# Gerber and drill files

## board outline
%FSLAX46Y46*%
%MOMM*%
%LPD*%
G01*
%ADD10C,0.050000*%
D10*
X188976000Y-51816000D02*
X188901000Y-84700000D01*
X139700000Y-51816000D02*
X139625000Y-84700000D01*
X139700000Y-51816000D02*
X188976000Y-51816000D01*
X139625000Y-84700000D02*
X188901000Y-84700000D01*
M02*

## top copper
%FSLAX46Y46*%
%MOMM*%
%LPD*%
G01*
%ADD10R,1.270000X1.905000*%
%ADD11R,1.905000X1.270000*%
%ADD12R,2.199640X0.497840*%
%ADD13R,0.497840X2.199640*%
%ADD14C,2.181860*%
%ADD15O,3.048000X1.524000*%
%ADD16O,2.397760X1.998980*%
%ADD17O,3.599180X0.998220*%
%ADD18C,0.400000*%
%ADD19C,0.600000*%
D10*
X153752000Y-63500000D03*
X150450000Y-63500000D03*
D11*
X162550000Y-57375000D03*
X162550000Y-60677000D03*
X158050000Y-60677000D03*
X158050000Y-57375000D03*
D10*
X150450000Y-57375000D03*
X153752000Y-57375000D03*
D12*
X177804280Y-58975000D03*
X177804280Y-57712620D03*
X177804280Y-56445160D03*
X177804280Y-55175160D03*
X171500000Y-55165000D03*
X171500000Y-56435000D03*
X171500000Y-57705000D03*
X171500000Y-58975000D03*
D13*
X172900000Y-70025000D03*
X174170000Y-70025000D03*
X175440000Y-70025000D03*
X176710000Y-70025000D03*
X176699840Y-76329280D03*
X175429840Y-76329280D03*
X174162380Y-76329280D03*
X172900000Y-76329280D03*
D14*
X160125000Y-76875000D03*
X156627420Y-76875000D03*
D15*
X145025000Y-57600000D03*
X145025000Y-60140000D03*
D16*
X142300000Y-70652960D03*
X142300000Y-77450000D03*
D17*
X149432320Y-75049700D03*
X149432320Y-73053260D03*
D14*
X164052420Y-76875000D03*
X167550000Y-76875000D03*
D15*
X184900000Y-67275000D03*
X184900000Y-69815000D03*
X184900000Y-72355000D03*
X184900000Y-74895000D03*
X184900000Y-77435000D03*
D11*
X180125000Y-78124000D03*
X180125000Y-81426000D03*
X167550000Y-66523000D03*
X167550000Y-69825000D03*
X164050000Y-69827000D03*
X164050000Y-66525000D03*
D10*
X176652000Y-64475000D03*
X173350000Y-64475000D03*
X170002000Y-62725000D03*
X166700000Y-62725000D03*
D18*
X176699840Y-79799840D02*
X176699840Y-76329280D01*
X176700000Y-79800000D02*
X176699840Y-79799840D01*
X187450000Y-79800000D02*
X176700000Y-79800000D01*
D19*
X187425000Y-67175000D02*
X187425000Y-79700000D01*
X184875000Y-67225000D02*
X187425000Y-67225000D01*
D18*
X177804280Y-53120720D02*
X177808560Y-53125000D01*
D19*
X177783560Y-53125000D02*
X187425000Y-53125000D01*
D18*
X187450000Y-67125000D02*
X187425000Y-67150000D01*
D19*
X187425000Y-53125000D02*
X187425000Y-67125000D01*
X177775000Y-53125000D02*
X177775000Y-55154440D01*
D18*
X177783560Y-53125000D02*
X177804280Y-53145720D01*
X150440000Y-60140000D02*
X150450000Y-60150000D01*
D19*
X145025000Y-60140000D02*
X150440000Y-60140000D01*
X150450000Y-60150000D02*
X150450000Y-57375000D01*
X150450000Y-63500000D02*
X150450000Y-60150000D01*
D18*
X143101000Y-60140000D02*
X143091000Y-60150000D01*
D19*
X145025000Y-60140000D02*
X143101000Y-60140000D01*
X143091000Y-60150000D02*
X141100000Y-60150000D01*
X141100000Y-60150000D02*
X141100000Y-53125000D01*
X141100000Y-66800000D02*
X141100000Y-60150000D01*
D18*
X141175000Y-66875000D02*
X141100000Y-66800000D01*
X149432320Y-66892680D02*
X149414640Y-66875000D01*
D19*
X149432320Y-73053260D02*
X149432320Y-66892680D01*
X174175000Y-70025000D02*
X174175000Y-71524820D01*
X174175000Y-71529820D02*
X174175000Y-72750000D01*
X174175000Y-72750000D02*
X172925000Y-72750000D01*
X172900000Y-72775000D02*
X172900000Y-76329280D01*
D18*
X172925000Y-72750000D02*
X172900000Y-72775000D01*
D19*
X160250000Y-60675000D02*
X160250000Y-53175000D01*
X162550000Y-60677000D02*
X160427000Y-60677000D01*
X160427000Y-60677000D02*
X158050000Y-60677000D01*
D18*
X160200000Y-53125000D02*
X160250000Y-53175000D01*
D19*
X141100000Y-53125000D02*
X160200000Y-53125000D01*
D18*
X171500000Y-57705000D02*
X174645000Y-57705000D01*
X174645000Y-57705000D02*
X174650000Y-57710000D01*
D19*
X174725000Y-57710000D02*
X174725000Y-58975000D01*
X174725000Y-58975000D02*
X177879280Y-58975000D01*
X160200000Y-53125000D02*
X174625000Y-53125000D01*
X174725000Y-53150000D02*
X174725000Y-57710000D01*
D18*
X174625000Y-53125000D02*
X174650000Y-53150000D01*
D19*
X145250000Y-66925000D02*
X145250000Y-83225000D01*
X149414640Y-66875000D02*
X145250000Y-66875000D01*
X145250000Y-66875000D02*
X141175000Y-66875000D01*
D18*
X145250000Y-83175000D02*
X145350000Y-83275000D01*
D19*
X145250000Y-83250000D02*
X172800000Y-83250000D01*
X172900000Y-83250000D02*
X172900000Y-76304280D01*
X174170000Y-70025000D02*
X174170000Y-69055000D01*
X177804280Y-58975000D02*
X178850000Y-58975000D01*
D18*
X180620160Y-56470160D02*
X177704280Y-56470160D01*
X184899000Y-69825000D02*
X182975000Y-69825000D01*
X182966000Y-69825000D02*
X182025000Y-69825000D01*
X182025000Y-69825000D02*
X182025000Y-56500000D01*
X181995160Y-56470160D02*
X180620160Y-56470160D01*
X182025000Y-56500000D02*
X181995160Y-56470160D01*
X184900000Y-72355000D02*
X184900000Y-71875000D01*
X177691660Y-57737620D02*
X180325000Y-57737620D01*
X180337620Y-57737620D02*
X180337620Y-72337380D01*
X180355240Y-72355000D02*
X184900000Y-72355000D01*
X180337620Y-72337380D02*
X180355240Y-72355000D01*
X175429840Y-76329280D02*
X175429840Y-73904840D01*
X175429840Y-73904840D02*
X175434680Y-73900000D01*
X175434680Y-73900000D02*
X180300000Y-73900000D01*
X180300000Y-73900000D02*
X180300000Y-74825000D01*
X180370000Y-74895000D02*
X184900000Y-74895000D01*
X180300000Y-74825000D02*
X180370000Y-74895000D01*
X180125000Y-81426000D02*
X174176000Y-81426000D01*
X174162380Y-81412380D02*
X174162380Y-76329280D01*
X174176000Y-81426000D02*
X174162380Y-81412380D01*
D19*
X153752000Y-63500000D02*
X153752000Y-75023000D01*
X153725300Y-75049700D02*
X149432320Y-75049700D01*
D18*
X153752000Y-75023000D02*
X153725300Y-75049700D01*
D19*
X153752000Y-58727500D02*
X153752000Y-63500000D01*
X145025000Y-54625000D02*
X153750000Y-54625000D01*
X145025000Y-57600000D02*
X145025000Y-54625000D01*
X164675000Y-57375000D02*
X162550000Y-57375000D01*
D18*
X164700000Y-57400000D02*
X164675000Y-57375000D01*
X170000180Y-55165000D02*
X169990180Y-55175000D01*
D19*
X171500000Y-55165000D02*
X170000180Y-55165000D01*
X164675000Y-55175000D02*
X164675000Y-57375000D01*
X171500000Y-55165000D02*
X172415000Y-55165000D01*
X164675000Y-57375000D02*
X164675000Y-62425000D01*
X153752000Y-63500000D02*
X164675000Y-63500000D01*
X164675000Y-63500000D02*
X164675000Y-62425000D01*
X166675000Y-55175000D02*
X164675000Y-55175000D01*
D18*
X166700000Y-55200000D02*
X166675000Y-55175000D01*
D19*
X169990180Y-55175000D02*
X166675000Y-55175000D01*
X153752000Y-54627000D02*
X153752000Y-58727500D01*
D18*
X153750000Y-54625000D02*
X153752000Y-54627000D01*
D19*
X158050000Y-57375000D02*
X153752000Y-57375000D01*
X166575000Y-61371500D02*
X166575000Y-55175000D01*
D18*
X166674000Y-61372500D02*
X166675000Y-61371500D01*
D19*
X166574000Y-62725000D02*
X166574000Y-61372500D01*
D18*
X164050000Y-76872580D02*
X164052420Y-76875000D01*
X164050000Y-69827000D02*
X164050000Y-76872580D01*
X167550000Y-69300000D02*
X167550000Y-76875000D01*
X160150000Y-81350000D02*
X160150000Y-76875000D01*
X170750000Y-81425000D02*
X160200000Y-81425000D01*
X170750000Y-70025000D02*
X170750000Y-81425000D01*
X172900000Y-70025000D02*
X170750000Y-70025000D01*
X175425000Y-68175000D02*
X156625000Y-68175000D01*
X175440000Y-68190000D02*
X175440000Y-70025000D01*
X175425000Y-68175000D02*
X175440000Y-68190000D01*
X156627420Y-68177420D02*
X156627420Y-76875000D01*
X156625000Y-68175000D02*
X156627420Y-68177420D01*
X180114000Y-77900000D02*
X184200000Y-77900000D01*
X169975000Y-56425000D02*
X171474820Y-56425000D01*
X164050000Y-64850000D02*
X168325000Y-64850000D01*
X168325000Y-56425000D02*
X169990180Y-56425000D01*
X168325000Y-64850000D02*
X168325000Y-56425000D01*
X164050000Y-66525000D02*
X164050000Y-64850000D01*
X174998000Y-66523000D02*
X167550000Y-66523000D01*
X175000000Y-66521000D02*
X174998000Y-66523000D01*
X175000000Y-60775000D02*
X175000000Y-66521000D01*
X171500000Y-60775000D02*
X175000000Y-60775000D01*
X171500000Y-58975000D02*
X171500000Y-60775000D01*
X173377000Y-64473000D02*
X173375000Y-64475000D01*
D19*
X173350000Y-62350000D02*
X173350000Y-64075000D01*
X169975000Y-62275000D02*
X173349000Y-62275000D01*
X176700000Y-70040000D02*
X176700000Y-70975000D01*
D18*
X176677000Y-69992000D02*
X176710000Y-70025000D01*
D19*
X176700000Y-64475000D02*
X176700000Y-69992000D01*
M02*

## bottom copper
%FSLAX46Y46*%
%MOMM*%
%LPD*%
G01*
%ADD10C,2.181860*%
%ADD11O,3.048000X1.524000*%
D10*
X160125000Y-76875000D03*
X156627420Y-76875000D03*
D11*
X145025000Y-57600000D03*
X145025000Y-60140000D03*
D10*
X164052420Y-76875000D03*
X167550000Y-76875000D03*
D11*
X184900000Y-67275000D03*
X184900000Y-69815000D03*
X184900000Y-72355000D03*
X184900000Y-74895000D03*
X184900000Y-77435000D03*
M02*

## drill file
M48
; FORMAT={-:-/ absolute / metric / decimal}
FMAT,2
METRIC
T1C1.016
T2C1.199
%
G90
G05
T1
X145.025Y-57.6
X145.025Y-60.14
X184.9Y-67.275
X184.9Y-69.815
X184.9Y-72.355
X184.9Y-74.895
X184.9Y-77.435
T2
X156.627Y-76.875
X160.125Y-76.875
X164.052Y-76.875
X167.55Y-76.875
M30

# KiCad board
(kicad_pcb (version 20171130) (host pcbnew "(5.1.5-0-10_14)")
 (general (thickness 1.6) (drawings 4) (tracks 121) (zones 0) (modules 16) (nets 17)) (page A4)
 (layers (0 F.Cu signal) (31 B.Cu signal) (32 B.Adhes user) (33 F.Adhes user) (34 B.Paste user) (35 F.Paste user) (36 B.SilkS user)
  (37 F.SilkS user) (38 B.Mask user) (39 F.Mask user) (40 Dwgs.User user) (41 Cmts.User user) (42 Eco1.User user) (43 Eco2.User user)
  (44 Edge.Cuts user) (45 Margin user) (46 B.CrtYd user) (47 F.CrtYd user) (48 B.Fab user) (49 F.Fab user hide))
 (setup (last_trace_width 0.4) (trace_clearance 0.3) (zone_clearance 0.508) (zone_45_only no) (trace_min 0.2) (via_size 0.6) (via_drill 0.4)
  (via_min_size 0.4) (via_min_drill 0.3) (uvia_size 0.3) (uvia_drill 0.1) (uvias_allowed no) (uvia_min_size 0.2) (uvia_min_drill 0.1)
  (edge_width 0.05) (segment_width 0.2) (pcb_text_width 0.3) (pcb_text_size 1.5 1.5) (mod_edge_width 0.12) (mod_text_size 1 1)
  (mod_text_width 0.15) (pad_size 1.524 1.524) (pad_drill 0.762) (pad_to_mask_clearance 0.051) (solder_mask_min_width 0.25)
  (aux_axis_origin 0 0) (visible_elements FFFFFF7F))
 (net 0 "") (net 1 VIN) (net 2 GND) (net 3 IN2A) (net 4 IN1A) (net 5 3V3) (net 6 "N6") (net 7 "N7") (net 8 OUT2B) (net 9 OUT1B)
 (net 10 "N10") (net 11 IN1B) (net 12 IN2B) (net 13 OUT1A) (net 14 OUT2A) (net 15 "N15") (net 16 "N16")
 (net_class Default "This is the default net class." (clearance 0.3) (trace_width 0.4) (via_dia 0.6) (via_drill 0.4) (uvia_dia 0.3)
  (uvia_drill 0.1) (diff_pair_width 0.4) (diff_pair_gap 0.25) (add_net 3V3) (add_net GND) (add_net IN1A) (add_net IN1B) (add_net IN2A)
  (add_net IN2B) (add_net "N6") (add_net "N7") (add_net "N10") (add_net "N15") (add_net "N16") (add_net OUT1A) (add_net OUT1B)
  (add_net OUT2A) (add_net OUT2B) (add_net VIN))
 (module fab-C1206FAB (layer F.Cu) (at 152.101 63.5 180)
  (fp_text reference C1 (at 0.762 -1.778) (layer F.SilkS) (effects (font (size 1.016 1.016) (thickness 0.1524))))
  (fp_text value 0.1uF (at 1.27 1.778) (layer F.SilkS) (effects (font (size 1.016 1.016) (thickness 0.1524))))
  (pad 1 smd rect (at -1.651 0 180) (size 1.27 1.905) (layers F.Cu F.Paste F.Mask) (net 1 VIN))
  (pad 2 smd rect (at 1.651 0 180) (size 1.27 1.905) (layers F.Cu F.Paste F.Mask) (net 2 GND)))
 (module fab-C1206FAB (layer F.Cu) (at 162.55 59.026 270)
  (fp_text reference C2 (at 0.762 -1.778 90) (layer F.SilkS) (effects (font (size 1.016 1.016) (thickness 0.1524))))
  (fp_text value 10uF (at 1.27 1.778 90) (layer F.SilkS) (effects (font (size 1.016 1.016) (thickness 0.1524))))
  (pad 1 smd rect (at -1.651 0 270) (size 1.27 1.905) (layers F.Cu F.Paste F.Mask) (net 1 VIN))
  (pad 2 smd rect (at 1.651 0 270) (size 1.27 1.905) (layers F.Cu F.Paste F.Mask) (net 2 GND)))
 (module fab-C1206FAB (layer F.Cu) (at 158.05 59.026 270)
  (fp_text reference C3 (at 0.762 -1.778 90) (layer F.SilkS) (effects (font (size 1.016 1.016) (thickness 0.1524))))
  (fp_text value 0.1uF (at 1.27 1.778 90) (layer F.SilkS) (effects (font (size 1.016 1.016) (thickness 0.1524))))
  (pad 2 smd rect (at 1.651 0 270) (size 1.27 1.905) (layers F.Cu F.Paste F.Mask) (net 2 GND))
  (pad 1 smd rect (at -1.651 0 270) (size 1.27 1.905) (layers F.Cu F.Paste F.Mask) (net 1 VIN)))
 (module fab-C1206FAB (layer F.Cu) (at 152.101 57.375 180)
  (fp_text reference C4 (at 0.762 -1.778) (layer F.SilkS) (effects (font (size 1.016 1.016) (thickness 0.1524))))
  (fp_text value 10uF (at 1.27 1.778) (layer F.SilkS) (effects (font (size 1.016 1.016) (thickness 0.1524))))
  (pad 2 smd rect (at 1.651 0 180) (size 1.27 1.905) (layers F.Cu F.Paste F.Mask) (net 2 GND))
  (pad 1 smd rect (at -1.651 0 180) (size 1.27 1.905) (layers F.Cu F.Paste F.Mask) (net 1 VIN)))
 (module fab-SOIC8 (layer F.Cu) (at 174.65214 57.07 90)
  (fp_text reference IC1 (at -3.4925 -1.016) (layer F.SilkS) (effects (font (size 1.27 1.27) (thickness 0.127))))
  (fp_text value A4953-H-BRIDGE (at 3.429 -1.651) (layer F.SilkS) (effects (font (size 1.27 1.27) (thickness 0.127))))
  (pad 1 smd rect (at -1.905 3.15214 90) (size 0.49784 2.19964) (layers F.Cu F.Paste F.Mask) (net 2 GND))
  (pad 2 smd rect (at -0.64262 3.15214 90) (size 0.49784 2.19964) (layers F.Cu F.Paste F.Mask) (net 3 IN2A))
  (pad 3 smd rect (at 0.62484 3.15214 90) (size 0.49784 2.19964) (layers F.Cu F.Paste F.Mask) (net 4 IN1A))
  (pad 4 smd rect (at 1.89484 3.15214 90) (size 0.49784 2.19964) (layers F.Cu F.Paste F.Mask) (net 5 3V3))
  (pad 5 smd rect (at 1.905 -3.15214 90) (size 0.49784 2.19964) (layers F.Cu F.Paste F.Mask) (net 1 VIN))
  (pad 6 smd rect (at 0.635 -3.15214 90) (size 0.49784 2.19964) (layers F.Cu F.Paste F.Mask) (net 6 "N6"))
  (pad 7 smd rect (at -0.635 -3.15214 90) (size 0.49784 2.19964) (layers F.Cu F.Paste F.Mask) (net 2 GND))
  (pad 8 smd rect (at -1.905 -3.15214 90) (size 0.49784 2.19964) (layers F.Cu F.Paste F.Mask) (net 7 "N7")))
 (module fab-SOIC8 (layer F.Cu) (at 174.805 73.17714)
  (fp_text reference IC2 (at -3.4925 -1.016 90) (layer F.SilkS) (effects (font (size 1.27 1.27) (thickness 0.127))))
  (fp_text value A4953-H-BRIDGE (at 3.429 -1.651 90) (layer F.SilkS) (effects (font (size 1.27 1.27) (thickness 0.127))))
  (pad 8 smd rect (at -1.905 -3.15214) (size 0.49784 2.19964) (layers F.Cu F.Paste F.Mask) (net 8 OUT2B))
  (pad 7 smd rect (at -0.635 -3.15214) (size 0.49784 2.19964) (layers F.Cu F.Paste F.Mask) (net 2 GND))
  (pad 6 smd rect (at 0.635 -3.15214) (size 0.49784 2.19964) (layers F.Cu F.Paste F.Mask) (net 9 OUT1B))
  (pad 5 smd rect (at 1.905 -3.15214) (size 0.49784 2.19964) (layers F.Cu F.Paste F.Mask) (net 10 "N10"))
  (pad 4 smd rect (at 1.89484 3.15214) (size 0.49784 2.19964) (layers F.Cu F.Paste F.Mask) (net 5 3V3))
  (pad 3 smd rect (at 0.62484 3.15214) (size 0.49784 2.19964) (layers F.Cu F.Paste F.Mask) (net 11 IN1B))
  (pad 2 smd rect (at -0.64262 3.15214) (size 0.49784 2.19964) (layers F.Cu F.Paste F.Mask) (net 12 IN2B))
  (pad 1 smd rect (at -1.905 3.15214) (size 0.49784 2.19964) (layers F.Cu F.Paste F.Mask) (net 2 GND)))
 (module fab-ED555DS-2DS (layer F.Cu) (at 158.32668 76.875)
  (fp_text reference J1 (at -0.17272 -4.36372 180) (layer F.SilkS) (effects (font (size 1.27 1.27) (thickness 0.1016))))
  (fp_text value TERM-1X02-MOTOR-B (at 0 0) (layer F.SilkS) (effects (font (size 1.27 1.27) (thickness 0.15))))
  (pad 1 thru_hole circle (at 1.79832 0) (size 2.18186 2.18186) (drill 1.19888) (layers F&B.Cu F.Paste F.SilkS F.Mask) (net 8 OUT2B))
  (pad 2 thru_hole circle (at -1.69926 0) (size 2.18186 2.18186) (drill 1.19888) (layers F&B.Cu F.Paste F.SilkS F.Mask) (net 9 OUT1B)))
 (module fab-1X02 (layer F.Cu) (at 145.025 58.87 270)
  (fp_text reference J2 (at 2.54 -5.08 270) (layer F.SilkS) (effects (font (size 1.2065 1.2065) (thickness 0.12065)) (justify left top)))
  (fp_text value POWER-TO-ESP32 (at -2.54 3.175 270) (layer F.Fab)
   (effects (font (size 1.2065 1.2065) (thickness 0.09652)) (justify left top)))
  (pad 1 thru_hole oval (at -1.27 0) (size 3.048 1.524) (drill 1.016) (layers *.Cu *.Mask) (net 1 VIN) (solder_mask_margin 0.1016))
  (pad 2 thru_hole oval (at 1.27 0) (size 3.048 1.524) (drill 1.016) (layers *.Cu *.Mask) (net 2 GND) (solder_mask_margin 0.1016)))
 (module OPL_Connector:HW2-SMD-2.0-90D (layer F.Cu) (at 144.47932 74.05148 270)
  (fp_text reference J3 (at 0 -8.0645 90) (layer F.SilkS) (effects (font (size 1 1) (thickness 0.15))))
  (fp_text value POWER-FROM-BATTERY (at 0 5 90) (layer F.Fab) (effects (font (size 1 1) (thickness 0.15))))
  (pad 3 smd oval (at -3.39852 2.17932) (size 2.39776 1.99898) (layers F.Cu F.Paste F.Mask))
  (pad 4 smd oval (at 3.39852 2.17932) (size 2.39776 1.99898) (layers F.Cu F.Paste F.Mask))
  (pad 2 smd oval (at 0.99822 -4.953) (size 3.59918 0.99822) (layers F.Cu F.Paste F.Mask) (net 1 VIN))
  (pad 1 smd oval (at -0.99822 -4.953) (size 3.59918 0.99822) (layers F.Cu F.Paste F.Mask) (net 2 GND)))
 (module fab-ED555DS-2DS (layer F.Cu) (at 165.75168 76.875)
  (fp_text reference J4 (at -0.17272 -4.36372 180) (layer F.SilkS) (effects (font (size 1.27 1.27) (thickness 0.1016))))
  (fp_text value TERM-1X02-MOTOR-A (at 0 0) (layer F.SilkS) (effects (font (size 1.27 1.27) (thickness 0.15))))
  (pad 2 thru_hole circle (at -1.69926 0) (size 2.18186 2.18186) (drill 1.19888) (layers F&B.Cu F.Paste F.SilkS F.Mask) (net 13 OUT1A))
  (pad 1 thru_hole circle (at 1.79832 0) (size 2.18186 2.18186) (drill 1.19888) (layers F&B.Cu F.Paste F.SilkS F.Mask) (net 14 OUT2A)))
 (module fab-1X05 (layer F.Cu) (at 184.9 72.355 270)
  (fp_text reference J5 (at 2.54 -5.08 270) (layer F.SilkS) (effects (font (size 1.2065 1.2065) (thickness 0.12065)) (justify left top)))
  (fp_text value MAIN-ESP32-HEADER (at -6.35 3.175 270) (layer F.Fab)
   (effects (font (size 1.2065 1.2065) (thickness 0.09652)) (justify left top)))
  (pad 1 thru_hole oval (at -5.08 0) (size 3.048 1.524) (drill 1.016) (layers *.Cu *.Mask) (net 5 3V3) (solder_mask_margin 0.1016))
  (pad 2 thru_hole oval (at -2.54 0) (size 3.048 1.524) (drill 1.016) (layers *.Cu *.Mask) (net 4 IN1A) (solder_mask_margin 0.1016))
  (pad 3 thru_hole oval (at 0 0) (size 3.048 1.524) (drill 1.016) (layers *.Cu *.Mask) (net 3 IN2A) (solder_mask_margin 0.1016))
  (pad 4 thru_hole oval (at 2.54 0) (size 3.048 1.524) (drill 1.016) (layers *.Cu *.Mask) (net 11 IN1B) (solder_mask_margin 0.1016))
  (pad 5 thru_hole oval (at 5.08 0) (size 3.048 1.524) (drill 1.016) (layers *.Cu *.Mask) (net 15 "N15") (solder_mask_margin 0.1016)))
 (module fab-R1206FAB (layer F.Cu) (at 180.125 79.775 270)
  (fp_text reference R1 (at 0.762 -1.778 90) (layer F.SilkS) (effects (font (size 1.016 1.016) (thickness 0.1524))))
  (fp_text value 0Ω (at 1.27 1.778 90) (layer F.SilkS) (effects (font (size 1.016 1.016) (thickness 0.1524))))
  (pad 1 smd rect (at -1.651 0 270) (size 1.27 1.905) (layers F.Cu F.Paste F.Mask) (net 15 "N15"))
  (pad 2 smd rect (at 1.651 0 270) (size 1.27 1.905) (layers F.Cu F.Paste F.Mask) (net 12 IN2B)))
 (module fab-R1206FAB (layer F.Cu) (at 167.55 68.174 270)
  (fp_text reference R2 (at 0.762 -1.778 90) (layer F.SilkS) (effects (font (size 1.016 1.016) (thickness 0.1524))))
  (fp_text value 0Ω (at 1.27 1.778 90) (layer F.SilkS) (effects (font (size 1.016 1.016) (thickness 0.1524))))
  (pad 1 smd rect (at -1.651 0 270) (size 1.27 1.905) (layers F.Cu F.Paste F.Mask) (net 7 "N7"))
  (pad 2 smd rect (at 1.651 0 270) (size 1.27 1.905) (layers F.Cu F.Paste F.Mask) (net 14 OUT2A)))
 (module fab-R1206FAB (layer F.Cu) (at 164.05 68.176 270)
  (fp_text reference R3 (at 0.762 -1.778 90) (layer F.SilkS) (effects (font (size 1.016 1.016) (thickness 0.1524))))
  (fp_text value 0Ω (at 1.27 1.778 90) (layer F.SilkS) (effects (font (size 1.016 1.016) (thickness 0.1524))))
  (pad 2 smd rect (at 1.651 0 270) (size 1.27 1.905) (layers F.Cu F.Paste F.Mask) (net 13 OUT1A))
  (pad 1 smd rect (at -1.651 0 270) (size 1.27 1.905) (layers F.Cu F.Paste F.Mask) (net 6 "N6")))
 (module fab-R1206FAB (layer F.Cu) (at 175.001 64.475 180)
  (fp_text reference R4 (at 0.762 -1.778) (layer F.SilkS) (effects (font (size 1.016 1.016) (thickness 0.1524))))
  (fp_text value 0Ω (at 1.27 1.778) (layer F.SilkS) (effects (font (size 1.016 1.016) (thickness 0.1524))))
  (pad 1 smd rect (at -1.651 0 180) (size 1.27 1.905) (layers F.Cu F.Paste F.Mask) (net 10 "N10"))
  (pad 2 smd rect (at 1.651 0 180) (size 1.27 1.905) (layers F.Cu F.Paste F.Mask) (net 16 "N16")))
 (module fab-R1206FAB (layer F.Cu) (at 168.351 62.725 180)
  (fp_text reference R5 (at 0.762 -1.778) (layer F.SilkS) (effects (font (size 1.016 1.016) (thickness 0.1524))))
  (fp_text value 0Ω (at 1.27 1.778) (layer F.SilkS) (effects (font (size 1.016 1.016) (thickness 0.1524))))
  (pad 1 smd rect (at -1.651 0 180) (size 1.27 1.905) (layers F.Cu F.Paste F.Mask) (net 16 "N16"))
  (pad 2 smd rect (at 1.651 0 180) (size 1.27 1.905) (layers F.Cu F.Paste F.Mask) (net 1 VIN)))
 (gr_line (start 188.976 51.816) (end 188.901 84.7) (layer Edge.Cuts) (width 0.05))
 (gr_line (start 139.7 51.816) (end 139.625 84.7) (layer Edge.Cuts) (width 0.05))
 (gr_line (start 139.7 51.816) (end 188.976 51.816) (layer Edge.Cuts) (width 0.05))
 (gr_line (start 139.625 84.7) (end 188.901 84.7) (layer Edge.Cuts) (width 0.05))
 (segment (start 176.69984 79.79984) (end 176.69984 76.32928) (width 0.4) (layer F.Cu) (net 5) (status 20))
 (segment (start 176.7 79.8) (end 176.69984 79.79984) (width 0.4) (layer F.Cu) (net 5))
 (segment (start 187.45 79.8) (end 176.7 79.8) (width 0.4) (layer F.Cu) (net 5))
 (segment (start 187.425 67.175) (end 187.425 79.7) (width 0.6) (layer F.Cu) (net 5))
 (segment (start 184.875 67.225) (end 187.425 67.225) (width 0.6) (layer F.Cu) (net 5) (status 10))
 (segment (start 177.80428 53.12072) (end 177.80856 53.125) (width 0.4) (layer F.Cu) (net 5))
 (segment (start 177.78356 53.125) (end 187.425 53.125) (width 0.6) (layer F.Cu) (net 5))
 (segment (start 187.45 67.125) (end 187.425 67.15) (width 0.4) (layer F.Cu) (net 5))
 (segment (start 187.425 53.125) (end 187.425 67.125) (width 0.6) (layer F.Cu) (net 5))
 (segment (start 177.775 53.125) (end 177.775 55.15444) (width 0.6) (layer F.Cu) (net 5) (status 20))
 (segment (start 177.78356 53.125) (end 177.80428 53.14572) (width 0.4) (layer F.Cu) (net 5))
 (segment (start 150.44 60.14) (end 150.45 60.15) (width 0.4) (layer F.Cu) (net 2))
 (segment (start 145.025 60.14) (end 150.44 60.14) (width 0.6) (layer F.Cu) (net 2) (status 10))
 (segment (start 150.45 60.15) (end 150.45 57.375) (width 0.6) (layer F.Cu) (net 2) (status 20))
 (segment (start 150.45 63.5) (end 150.45 60.15) (width 0.6) (layer F.Cu) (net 2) (status 10))
 (segment (start 143.101 60.14) (end 143.091 60.15) (width 0.4) (layer F.Cu) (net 2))
 (segment (start 145.025 60.14) (end 143.101 60.14) (width 0.6) (layer F.Cu) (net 2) (status 10))
 (segment (start 143.091 60.15) (end 141.1 60.15) (width 0.6) (layer F.Cu) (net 2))
 (segment (start 141.1 60.15) (end 141.1 53.125) (width 0.6) (layer F.Cu) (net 2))
 (segment (start 141.1 66.8) (end 141.1 60.15) (width 0.6) (layer F.Cu) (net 2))
 (segment (start 141.175 66.875) (end 141.1 66.8) (width 0.4) (layer F.Cu) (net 2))
 (segment (start 149.43232 66.89268) (end 149.41464 66.875) (width 0.4) (layer F.Cu) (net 2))
 (segment (start 149.43232 73.05326) (end 149.43232 66.89268) (width 0.6) (layer F.Cu) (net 2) (status 10))
 (segment (start 174.175 70.025) (end 174.175 71.52482) (width 0.6) (layer F.Cu) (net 2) (status 10))
 (segment (start 174.175 71.52982) (end 174.175 72.75) (width 0.6) (layer F.Cu) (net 2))
 (segment (start 174.175 72.75) (end 172.925 72.75) (width 0.6) (layer F.Cu) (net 2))
 (segment (start 172.9 72.775) (end 172.9 76.32928) (width 0.6) (layer F.Cu) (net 2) (status 20))
 (segment (start 172.925 72.75) (end 172.9 72.775) (width 0.4) (layer F.Cu) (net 2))
 (segment (start 160.25 60.675) (end 160.25 53.175) (width 0.6) (layer F.Cu) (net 2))
 (segment (start 162.55 60.677) (end 160.427 60.677) (width 0.6) (layer F.Cu) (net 2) (status 10))
 (segment (start 160.427 60.677) (end 158.05 60.677) (width 0.6) (layer F.Cu) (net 2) (status 20))
 (segment (start 160.2 53.125) (end 160.25 53.175) (width 0.4) (layer F.Cu) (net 2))
 (segment (start 141.1 53.125) (end 160.2 53.125) (width 0.6) (layer F.Cu) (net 2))
 (segment (start 171.5 57.705) (end 174.645 57.705) (width 0.4) (layer F.Cu) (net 2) (status 10))
 (segment (start 174.645 57.705) (end 174.65 57.71) (width 0.4) (layer F.Cu) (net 2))
 (segment (start 174.725 57.71) (end 174.725 58.975) (width 0.6) (layer F.Cu) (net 2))
 (segment (start 174.725 58.975) (end 177.87928 58.975) (width 0.6) (layer F.Cu) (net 2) (status 20))
 (segment (start 160.2 53.125) (end 174.625 53.125) (width 0.6) (layer F.Cu) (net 2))
 (segment (start 174.725 53.15) (end 174.725 57.71) (width 0.6) (layer F.Cu) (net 2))
 (segment (start 174.625 53.125) (end 174.65 53.15) (width 0.4) (layer F.Cu) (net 2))
 (segment (start 145.25 66.925) (end 145.25 83.225) (width 0.6) (layer F.Cu) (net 2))
 (segment (start 149.41464 66.875) (end 145.25 66.875) (width 0.6) (layer F.Cu) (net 2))
 (segment (start 145.25 66.875) (end 141.175 66.875) (width 0.6) (layer F.Cu) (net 2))
 (segment (start 145.25 83.175) (end 145.35 83.275) (width 0.4) (layer F.Cu) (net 2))
 (segment (start 145.25 83.25) (end 172.8 83.25) (width 0.6) (layer F.Cu) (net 2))
 (segment (start 172.9 83.25) (end 172.9 76.30428) (width 0.6) (layer F.Cu) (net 2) (status 20))
 (segment (start 174.17 70.025) (end 174.17 69.055) (width 0.6) (layer F.Cu) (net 2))
 (segment (start 177.80428 58.975) (end 178.85 58.975) (width 0.6) (layer F.Cu) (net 2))
 (segment (start 180.62016 56.47016) (end 177.70428 56.47016) (width 0.4) (layer F.Cu) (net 4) (status 20))
 (segment (start 184.899 69.825) (end 182.975 69.825) (width 0.4) (layer F.Cu) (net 4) (status 10))
 (segment (start 182.966 69.825) (end 182.025 69.825) (width 0.4) (layer F.Cu) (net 4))
 (segment (start 182.025 69.825) (end 182.025 56.5) (width 0.4) (layer F.Cu) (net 4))
 (segment (start 181.99516 56.47016) (end 180.62016 56.47016) (width 0.4) (layer F.Cu) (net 4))
 (segment (start 182.025 56.5) (end 181.99516 56.47016) (width 0.4) (layer F.Cu) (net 4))
 (segment (start 184.9 72.355) (end 184.9 71.875) (width 0.4) (layer F.Cu) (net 3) (status 30))
 (segment (start 177.69166 57.73762) (end 180.325 57.73762) (width 0.4) (layer F.Cu) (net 3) (status 10))
 (segment (start 180.33762 57.73762) (end 180.33762 72.33738) (width 0.4) (layer F.Cu) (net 3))
 (segment (start 180.35524 72.355) (end 184.9 72.355) (width 0.4) (layer F.Cu) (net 3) (status 20))
 (segment (start 180.33762 72.33738) (end 180.35524 72.355) (width 0.4) (layer F.Cu) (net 3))
 (segment (start 175.42984 76.32928) (end 175.42984 73.90484) (width 0.4) (layer F.Cu) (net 11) (status 10))
 (segment (start 175.42984 73.90484) (end 175.43468 73.9) (width 0.4) (layer F.Cu) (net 11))
 (segment (start 175.43468 73.9) (end 180.3 73.9) (width 0.4) (layer F.Cu) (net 11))
 (segment (start 180.3 73.9) (end 180.3 74.825) (width 0.4) (layer F.Cu) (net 11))
 (segment (start 180.37 74.895) (end 184.9 74.895) (width 0.4) (layer F.Cu) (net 11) (status 20))
 (segment (start 180.3 74.825) (end 180.37 74.895) (width 0.4) (layer F.Cu) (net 11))
 (segment (start 180.125 81.426) (end 174.176 81.426) (width 0.4) (layer F.Cu) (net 12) (status 10))
 (segment (start 174.16238 81.41238) (end 174.16238 76.32928) (width 0.4) (layer F.Cu) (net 12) (status 20))
 (segment (start 174.176 81.426) (end 174.16238 81.41238) (width 0.4) (layer F.Cu) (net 12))
 (segment (start 153.752 63.5) (end 153.752 75.023) (width 0.6) (layer F.Cu) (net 1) (status 10))
 (segment (start 153.7253 75.0497) (end 149.43232 75.0497) (width 0.6) (layer F.Cu) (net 1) (status 20))
 (segment (start 153.752 75.023) (end 153.7253 75.0497) (width 0.4) (layer F.Cu) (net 1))
 (segment (start 153.752 58.7275) (end 153.752 63.5) (width 0.6) (layer F.Cu) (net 1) (status 20))
 (segment (start 145.025 54.625) (end 153.75 54.625) (width 0.6) (layer F.Cu) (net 1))
 (segment (start 145.025 57.6) (end 145.025 54.625) (width 0.6) (layer F.Cu) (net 1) (status 10))
 (segment (start 164.675 57.375) (end 162.55 57.375) (width 0.6) (layer F.Cu) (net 1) (status 20))
 (segment (start 164.7 57.4) (end 164.675 57.375) (width 0.4) (layer F.Cu) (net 1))
 (segment (start 170.00018 55.165) (end 169.99018 55.175) (width 0.4) (layer F.Cu) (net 1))
 (segment (start 171.5 55.165) (end 170.00018 55.165) (width 0.6) (layer F.Cu) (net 1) (status 10))
 (segment (start 164.675 55.175) (end 164.675 57.375) (width 0.6) (layer F.Cu) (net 1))
 (segment (start 171.5 55.165) (end 172.415 55.165) (width 0.6) (layer F.Cu) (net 1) (status 30))
 (segment (start 164.675 57.375) (end 164.675 62.425) (width 0.6) (layer F.Cu) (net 1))
 (segment (start 153.752 63.5) (end 164.675 63.5) (width 0.6) (layer F.Cu) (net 1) (status 10))
 (segment (start 164.675 63.5) (end 164.675 62.425) (width 0.6) (layer F.Cu) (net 1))
 (segment (start 166.675 55.175) (end 164.675 55.175) (width 0.6) (layer F.Cu) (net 1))
 (segment (start 166.7 55.2) (end 166.675 55.175) (width 0.4) (layer F.Cu) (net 1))
 (segment (start 169.99018 55.175) (end 166.675 55.175) (width 0.6) (layer F.Cu) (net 1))
 (segment (start 153.752 54.627) (end 153.752 58.7275) (width 0.6) (layer F.Cu) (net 1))
 (segment (start 153.75 54.625) (end 153.752 54.627) (width 0.4) (layer F.Cu) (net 1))
 (segment (start 158.05 57.375) (end 153.752 57.375) (width 0.6) (layer F.Cu) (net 1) (status 30))
 (segment (start 166.575 61.3715) (end 166.575 55.175) (width 0.6) (layer F.Cu) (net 1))
 (segment (start 166.674 61.3725) (end 166.675 61.3715) (width 0.4) (layer F.Cu) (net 1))
 (segment (start 166.574 62.725) (end 166.574 61.3725) (width 0.6) (layer F.Cu) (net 1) (status 10))
 (segment (start 164.05 76.87258) (end 164.05242 76.875) (width 0.4) (layer F.Cu) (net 13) (status 30))
 (segment (start 164.05 69.827) (end 164.05 76.87258) (width 0.4) (layer F.Cu) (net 13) (status 30))
 (segment (start 167.55 69.3) (end 167.55 76.875) (width 0.4) (layer F.Cu) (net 14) (status 30))
 (segment (start 160.15 81.35) (end 160.15 76.875) (width 0.4) (layer F.Cu) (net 8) (status 20))
 (segment (start 170.75 81.425) (end 160.2 81.425) (width 0.4) (layer F.Cu) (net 8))
 (segment (start 170.75 70.025) (end 170.75 81.425) (width 0.4) (layer F.Cu) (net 8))
 (segment (start 172.9 70.025) (end 170.75 70.025) (width 0.4) (layer F.Cu) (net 8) (status 10))
 (segment (start 175.425 68.175) (end 156.625 68.175) (width 0.4) (layer F.Cu) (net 9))
 (segment (start 175.44 68.19) (end 175.44 70.025) (width 0.4) (layer F.Cu) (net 9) (status 20))
 (segment (start 175.425 68.175) (end 175.44 68.19) (width 0.4) (layer F.Cu) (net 9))
 (segment (start 156.62742 68.17742) (end 156.62742 76.875) (width 0.4) (layer F.Cu) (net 9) (status 20))
 (segment (start 156.625 68.175) (end 156.62742 68.17742) (width 0.4) (layer F.Cu) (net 9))
 (segment (start 180.114 77.9) (end 184.2 77.9) (width 0.4) (layer F.Cu) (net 15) (status 30))
 (segment (start 169.975 56.425) (end 171.47482 56.425) (width 0.4) (layer F.Cu) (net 6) (status 20))
 (segment (start 164.05 64.85) (end 168.325 64.85) (width 0.4) (layer F.Cu) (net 6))
 (segment (start 168.325 56.425) (end 169.99018 56.425) (width 0.4) (layer F.Cu) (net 6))
 (segment (start 168.325 64.85) (end 168.325 56.425) (width 0.4) (layer F.Cu) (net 6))
 (segment (start 164.05 66.525) (end 164.05 64.85) (width 0.4) (layer F.Cu) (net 6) (status 10))
 (segment (start 174.998 66.523) (end 167.55 66.523) (width 0.4) (layer F.Cu) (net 7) (status 20))
 (segment (start 175 66.521) (end 174.998 66.523) (width 0.4) (layer F.Cu) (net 7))
 (segment (start 175 60.775) (end 175 66.521) (width 0.4) (layer F.Cu) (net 7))
 (segment (start 171.5 60.775) (end 175 60.775) (width 0.4) (layer F.Cu) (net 7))
 (segment (start 171.5 58.975) (end 171.5 60.775) (width 0.4) (layer F.Cu) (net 7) (status 10))
 (segment (start 173.377 64.473) (end 173.375 64.475) (width 0.4) (layer F.Cu) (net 16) (status 30))
 (segment (start 173.35 62.35) (end 173.35 64.075) (width 0.6) (layer F.Cu) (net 16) (status 20))
 (segment (start 169.975 62.275) (end 173.349 62.275) (width 0.6) (layer F.Cu) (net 16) (status 10))
 (segment (start 176.7 70.04) (end 176.7 70.975) (width 0.6) (layer F.Cu) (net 10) (status 30))
 (segment (start 176.677 69.992) (end 176.71 70.025) (width 0.4) (layer F.Cu) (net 10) (status 30))
 (segment (start 176.7 64.475) (end 176.7 69.992) (width 0.6) (layer F.Cu) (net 10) (status 30)))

